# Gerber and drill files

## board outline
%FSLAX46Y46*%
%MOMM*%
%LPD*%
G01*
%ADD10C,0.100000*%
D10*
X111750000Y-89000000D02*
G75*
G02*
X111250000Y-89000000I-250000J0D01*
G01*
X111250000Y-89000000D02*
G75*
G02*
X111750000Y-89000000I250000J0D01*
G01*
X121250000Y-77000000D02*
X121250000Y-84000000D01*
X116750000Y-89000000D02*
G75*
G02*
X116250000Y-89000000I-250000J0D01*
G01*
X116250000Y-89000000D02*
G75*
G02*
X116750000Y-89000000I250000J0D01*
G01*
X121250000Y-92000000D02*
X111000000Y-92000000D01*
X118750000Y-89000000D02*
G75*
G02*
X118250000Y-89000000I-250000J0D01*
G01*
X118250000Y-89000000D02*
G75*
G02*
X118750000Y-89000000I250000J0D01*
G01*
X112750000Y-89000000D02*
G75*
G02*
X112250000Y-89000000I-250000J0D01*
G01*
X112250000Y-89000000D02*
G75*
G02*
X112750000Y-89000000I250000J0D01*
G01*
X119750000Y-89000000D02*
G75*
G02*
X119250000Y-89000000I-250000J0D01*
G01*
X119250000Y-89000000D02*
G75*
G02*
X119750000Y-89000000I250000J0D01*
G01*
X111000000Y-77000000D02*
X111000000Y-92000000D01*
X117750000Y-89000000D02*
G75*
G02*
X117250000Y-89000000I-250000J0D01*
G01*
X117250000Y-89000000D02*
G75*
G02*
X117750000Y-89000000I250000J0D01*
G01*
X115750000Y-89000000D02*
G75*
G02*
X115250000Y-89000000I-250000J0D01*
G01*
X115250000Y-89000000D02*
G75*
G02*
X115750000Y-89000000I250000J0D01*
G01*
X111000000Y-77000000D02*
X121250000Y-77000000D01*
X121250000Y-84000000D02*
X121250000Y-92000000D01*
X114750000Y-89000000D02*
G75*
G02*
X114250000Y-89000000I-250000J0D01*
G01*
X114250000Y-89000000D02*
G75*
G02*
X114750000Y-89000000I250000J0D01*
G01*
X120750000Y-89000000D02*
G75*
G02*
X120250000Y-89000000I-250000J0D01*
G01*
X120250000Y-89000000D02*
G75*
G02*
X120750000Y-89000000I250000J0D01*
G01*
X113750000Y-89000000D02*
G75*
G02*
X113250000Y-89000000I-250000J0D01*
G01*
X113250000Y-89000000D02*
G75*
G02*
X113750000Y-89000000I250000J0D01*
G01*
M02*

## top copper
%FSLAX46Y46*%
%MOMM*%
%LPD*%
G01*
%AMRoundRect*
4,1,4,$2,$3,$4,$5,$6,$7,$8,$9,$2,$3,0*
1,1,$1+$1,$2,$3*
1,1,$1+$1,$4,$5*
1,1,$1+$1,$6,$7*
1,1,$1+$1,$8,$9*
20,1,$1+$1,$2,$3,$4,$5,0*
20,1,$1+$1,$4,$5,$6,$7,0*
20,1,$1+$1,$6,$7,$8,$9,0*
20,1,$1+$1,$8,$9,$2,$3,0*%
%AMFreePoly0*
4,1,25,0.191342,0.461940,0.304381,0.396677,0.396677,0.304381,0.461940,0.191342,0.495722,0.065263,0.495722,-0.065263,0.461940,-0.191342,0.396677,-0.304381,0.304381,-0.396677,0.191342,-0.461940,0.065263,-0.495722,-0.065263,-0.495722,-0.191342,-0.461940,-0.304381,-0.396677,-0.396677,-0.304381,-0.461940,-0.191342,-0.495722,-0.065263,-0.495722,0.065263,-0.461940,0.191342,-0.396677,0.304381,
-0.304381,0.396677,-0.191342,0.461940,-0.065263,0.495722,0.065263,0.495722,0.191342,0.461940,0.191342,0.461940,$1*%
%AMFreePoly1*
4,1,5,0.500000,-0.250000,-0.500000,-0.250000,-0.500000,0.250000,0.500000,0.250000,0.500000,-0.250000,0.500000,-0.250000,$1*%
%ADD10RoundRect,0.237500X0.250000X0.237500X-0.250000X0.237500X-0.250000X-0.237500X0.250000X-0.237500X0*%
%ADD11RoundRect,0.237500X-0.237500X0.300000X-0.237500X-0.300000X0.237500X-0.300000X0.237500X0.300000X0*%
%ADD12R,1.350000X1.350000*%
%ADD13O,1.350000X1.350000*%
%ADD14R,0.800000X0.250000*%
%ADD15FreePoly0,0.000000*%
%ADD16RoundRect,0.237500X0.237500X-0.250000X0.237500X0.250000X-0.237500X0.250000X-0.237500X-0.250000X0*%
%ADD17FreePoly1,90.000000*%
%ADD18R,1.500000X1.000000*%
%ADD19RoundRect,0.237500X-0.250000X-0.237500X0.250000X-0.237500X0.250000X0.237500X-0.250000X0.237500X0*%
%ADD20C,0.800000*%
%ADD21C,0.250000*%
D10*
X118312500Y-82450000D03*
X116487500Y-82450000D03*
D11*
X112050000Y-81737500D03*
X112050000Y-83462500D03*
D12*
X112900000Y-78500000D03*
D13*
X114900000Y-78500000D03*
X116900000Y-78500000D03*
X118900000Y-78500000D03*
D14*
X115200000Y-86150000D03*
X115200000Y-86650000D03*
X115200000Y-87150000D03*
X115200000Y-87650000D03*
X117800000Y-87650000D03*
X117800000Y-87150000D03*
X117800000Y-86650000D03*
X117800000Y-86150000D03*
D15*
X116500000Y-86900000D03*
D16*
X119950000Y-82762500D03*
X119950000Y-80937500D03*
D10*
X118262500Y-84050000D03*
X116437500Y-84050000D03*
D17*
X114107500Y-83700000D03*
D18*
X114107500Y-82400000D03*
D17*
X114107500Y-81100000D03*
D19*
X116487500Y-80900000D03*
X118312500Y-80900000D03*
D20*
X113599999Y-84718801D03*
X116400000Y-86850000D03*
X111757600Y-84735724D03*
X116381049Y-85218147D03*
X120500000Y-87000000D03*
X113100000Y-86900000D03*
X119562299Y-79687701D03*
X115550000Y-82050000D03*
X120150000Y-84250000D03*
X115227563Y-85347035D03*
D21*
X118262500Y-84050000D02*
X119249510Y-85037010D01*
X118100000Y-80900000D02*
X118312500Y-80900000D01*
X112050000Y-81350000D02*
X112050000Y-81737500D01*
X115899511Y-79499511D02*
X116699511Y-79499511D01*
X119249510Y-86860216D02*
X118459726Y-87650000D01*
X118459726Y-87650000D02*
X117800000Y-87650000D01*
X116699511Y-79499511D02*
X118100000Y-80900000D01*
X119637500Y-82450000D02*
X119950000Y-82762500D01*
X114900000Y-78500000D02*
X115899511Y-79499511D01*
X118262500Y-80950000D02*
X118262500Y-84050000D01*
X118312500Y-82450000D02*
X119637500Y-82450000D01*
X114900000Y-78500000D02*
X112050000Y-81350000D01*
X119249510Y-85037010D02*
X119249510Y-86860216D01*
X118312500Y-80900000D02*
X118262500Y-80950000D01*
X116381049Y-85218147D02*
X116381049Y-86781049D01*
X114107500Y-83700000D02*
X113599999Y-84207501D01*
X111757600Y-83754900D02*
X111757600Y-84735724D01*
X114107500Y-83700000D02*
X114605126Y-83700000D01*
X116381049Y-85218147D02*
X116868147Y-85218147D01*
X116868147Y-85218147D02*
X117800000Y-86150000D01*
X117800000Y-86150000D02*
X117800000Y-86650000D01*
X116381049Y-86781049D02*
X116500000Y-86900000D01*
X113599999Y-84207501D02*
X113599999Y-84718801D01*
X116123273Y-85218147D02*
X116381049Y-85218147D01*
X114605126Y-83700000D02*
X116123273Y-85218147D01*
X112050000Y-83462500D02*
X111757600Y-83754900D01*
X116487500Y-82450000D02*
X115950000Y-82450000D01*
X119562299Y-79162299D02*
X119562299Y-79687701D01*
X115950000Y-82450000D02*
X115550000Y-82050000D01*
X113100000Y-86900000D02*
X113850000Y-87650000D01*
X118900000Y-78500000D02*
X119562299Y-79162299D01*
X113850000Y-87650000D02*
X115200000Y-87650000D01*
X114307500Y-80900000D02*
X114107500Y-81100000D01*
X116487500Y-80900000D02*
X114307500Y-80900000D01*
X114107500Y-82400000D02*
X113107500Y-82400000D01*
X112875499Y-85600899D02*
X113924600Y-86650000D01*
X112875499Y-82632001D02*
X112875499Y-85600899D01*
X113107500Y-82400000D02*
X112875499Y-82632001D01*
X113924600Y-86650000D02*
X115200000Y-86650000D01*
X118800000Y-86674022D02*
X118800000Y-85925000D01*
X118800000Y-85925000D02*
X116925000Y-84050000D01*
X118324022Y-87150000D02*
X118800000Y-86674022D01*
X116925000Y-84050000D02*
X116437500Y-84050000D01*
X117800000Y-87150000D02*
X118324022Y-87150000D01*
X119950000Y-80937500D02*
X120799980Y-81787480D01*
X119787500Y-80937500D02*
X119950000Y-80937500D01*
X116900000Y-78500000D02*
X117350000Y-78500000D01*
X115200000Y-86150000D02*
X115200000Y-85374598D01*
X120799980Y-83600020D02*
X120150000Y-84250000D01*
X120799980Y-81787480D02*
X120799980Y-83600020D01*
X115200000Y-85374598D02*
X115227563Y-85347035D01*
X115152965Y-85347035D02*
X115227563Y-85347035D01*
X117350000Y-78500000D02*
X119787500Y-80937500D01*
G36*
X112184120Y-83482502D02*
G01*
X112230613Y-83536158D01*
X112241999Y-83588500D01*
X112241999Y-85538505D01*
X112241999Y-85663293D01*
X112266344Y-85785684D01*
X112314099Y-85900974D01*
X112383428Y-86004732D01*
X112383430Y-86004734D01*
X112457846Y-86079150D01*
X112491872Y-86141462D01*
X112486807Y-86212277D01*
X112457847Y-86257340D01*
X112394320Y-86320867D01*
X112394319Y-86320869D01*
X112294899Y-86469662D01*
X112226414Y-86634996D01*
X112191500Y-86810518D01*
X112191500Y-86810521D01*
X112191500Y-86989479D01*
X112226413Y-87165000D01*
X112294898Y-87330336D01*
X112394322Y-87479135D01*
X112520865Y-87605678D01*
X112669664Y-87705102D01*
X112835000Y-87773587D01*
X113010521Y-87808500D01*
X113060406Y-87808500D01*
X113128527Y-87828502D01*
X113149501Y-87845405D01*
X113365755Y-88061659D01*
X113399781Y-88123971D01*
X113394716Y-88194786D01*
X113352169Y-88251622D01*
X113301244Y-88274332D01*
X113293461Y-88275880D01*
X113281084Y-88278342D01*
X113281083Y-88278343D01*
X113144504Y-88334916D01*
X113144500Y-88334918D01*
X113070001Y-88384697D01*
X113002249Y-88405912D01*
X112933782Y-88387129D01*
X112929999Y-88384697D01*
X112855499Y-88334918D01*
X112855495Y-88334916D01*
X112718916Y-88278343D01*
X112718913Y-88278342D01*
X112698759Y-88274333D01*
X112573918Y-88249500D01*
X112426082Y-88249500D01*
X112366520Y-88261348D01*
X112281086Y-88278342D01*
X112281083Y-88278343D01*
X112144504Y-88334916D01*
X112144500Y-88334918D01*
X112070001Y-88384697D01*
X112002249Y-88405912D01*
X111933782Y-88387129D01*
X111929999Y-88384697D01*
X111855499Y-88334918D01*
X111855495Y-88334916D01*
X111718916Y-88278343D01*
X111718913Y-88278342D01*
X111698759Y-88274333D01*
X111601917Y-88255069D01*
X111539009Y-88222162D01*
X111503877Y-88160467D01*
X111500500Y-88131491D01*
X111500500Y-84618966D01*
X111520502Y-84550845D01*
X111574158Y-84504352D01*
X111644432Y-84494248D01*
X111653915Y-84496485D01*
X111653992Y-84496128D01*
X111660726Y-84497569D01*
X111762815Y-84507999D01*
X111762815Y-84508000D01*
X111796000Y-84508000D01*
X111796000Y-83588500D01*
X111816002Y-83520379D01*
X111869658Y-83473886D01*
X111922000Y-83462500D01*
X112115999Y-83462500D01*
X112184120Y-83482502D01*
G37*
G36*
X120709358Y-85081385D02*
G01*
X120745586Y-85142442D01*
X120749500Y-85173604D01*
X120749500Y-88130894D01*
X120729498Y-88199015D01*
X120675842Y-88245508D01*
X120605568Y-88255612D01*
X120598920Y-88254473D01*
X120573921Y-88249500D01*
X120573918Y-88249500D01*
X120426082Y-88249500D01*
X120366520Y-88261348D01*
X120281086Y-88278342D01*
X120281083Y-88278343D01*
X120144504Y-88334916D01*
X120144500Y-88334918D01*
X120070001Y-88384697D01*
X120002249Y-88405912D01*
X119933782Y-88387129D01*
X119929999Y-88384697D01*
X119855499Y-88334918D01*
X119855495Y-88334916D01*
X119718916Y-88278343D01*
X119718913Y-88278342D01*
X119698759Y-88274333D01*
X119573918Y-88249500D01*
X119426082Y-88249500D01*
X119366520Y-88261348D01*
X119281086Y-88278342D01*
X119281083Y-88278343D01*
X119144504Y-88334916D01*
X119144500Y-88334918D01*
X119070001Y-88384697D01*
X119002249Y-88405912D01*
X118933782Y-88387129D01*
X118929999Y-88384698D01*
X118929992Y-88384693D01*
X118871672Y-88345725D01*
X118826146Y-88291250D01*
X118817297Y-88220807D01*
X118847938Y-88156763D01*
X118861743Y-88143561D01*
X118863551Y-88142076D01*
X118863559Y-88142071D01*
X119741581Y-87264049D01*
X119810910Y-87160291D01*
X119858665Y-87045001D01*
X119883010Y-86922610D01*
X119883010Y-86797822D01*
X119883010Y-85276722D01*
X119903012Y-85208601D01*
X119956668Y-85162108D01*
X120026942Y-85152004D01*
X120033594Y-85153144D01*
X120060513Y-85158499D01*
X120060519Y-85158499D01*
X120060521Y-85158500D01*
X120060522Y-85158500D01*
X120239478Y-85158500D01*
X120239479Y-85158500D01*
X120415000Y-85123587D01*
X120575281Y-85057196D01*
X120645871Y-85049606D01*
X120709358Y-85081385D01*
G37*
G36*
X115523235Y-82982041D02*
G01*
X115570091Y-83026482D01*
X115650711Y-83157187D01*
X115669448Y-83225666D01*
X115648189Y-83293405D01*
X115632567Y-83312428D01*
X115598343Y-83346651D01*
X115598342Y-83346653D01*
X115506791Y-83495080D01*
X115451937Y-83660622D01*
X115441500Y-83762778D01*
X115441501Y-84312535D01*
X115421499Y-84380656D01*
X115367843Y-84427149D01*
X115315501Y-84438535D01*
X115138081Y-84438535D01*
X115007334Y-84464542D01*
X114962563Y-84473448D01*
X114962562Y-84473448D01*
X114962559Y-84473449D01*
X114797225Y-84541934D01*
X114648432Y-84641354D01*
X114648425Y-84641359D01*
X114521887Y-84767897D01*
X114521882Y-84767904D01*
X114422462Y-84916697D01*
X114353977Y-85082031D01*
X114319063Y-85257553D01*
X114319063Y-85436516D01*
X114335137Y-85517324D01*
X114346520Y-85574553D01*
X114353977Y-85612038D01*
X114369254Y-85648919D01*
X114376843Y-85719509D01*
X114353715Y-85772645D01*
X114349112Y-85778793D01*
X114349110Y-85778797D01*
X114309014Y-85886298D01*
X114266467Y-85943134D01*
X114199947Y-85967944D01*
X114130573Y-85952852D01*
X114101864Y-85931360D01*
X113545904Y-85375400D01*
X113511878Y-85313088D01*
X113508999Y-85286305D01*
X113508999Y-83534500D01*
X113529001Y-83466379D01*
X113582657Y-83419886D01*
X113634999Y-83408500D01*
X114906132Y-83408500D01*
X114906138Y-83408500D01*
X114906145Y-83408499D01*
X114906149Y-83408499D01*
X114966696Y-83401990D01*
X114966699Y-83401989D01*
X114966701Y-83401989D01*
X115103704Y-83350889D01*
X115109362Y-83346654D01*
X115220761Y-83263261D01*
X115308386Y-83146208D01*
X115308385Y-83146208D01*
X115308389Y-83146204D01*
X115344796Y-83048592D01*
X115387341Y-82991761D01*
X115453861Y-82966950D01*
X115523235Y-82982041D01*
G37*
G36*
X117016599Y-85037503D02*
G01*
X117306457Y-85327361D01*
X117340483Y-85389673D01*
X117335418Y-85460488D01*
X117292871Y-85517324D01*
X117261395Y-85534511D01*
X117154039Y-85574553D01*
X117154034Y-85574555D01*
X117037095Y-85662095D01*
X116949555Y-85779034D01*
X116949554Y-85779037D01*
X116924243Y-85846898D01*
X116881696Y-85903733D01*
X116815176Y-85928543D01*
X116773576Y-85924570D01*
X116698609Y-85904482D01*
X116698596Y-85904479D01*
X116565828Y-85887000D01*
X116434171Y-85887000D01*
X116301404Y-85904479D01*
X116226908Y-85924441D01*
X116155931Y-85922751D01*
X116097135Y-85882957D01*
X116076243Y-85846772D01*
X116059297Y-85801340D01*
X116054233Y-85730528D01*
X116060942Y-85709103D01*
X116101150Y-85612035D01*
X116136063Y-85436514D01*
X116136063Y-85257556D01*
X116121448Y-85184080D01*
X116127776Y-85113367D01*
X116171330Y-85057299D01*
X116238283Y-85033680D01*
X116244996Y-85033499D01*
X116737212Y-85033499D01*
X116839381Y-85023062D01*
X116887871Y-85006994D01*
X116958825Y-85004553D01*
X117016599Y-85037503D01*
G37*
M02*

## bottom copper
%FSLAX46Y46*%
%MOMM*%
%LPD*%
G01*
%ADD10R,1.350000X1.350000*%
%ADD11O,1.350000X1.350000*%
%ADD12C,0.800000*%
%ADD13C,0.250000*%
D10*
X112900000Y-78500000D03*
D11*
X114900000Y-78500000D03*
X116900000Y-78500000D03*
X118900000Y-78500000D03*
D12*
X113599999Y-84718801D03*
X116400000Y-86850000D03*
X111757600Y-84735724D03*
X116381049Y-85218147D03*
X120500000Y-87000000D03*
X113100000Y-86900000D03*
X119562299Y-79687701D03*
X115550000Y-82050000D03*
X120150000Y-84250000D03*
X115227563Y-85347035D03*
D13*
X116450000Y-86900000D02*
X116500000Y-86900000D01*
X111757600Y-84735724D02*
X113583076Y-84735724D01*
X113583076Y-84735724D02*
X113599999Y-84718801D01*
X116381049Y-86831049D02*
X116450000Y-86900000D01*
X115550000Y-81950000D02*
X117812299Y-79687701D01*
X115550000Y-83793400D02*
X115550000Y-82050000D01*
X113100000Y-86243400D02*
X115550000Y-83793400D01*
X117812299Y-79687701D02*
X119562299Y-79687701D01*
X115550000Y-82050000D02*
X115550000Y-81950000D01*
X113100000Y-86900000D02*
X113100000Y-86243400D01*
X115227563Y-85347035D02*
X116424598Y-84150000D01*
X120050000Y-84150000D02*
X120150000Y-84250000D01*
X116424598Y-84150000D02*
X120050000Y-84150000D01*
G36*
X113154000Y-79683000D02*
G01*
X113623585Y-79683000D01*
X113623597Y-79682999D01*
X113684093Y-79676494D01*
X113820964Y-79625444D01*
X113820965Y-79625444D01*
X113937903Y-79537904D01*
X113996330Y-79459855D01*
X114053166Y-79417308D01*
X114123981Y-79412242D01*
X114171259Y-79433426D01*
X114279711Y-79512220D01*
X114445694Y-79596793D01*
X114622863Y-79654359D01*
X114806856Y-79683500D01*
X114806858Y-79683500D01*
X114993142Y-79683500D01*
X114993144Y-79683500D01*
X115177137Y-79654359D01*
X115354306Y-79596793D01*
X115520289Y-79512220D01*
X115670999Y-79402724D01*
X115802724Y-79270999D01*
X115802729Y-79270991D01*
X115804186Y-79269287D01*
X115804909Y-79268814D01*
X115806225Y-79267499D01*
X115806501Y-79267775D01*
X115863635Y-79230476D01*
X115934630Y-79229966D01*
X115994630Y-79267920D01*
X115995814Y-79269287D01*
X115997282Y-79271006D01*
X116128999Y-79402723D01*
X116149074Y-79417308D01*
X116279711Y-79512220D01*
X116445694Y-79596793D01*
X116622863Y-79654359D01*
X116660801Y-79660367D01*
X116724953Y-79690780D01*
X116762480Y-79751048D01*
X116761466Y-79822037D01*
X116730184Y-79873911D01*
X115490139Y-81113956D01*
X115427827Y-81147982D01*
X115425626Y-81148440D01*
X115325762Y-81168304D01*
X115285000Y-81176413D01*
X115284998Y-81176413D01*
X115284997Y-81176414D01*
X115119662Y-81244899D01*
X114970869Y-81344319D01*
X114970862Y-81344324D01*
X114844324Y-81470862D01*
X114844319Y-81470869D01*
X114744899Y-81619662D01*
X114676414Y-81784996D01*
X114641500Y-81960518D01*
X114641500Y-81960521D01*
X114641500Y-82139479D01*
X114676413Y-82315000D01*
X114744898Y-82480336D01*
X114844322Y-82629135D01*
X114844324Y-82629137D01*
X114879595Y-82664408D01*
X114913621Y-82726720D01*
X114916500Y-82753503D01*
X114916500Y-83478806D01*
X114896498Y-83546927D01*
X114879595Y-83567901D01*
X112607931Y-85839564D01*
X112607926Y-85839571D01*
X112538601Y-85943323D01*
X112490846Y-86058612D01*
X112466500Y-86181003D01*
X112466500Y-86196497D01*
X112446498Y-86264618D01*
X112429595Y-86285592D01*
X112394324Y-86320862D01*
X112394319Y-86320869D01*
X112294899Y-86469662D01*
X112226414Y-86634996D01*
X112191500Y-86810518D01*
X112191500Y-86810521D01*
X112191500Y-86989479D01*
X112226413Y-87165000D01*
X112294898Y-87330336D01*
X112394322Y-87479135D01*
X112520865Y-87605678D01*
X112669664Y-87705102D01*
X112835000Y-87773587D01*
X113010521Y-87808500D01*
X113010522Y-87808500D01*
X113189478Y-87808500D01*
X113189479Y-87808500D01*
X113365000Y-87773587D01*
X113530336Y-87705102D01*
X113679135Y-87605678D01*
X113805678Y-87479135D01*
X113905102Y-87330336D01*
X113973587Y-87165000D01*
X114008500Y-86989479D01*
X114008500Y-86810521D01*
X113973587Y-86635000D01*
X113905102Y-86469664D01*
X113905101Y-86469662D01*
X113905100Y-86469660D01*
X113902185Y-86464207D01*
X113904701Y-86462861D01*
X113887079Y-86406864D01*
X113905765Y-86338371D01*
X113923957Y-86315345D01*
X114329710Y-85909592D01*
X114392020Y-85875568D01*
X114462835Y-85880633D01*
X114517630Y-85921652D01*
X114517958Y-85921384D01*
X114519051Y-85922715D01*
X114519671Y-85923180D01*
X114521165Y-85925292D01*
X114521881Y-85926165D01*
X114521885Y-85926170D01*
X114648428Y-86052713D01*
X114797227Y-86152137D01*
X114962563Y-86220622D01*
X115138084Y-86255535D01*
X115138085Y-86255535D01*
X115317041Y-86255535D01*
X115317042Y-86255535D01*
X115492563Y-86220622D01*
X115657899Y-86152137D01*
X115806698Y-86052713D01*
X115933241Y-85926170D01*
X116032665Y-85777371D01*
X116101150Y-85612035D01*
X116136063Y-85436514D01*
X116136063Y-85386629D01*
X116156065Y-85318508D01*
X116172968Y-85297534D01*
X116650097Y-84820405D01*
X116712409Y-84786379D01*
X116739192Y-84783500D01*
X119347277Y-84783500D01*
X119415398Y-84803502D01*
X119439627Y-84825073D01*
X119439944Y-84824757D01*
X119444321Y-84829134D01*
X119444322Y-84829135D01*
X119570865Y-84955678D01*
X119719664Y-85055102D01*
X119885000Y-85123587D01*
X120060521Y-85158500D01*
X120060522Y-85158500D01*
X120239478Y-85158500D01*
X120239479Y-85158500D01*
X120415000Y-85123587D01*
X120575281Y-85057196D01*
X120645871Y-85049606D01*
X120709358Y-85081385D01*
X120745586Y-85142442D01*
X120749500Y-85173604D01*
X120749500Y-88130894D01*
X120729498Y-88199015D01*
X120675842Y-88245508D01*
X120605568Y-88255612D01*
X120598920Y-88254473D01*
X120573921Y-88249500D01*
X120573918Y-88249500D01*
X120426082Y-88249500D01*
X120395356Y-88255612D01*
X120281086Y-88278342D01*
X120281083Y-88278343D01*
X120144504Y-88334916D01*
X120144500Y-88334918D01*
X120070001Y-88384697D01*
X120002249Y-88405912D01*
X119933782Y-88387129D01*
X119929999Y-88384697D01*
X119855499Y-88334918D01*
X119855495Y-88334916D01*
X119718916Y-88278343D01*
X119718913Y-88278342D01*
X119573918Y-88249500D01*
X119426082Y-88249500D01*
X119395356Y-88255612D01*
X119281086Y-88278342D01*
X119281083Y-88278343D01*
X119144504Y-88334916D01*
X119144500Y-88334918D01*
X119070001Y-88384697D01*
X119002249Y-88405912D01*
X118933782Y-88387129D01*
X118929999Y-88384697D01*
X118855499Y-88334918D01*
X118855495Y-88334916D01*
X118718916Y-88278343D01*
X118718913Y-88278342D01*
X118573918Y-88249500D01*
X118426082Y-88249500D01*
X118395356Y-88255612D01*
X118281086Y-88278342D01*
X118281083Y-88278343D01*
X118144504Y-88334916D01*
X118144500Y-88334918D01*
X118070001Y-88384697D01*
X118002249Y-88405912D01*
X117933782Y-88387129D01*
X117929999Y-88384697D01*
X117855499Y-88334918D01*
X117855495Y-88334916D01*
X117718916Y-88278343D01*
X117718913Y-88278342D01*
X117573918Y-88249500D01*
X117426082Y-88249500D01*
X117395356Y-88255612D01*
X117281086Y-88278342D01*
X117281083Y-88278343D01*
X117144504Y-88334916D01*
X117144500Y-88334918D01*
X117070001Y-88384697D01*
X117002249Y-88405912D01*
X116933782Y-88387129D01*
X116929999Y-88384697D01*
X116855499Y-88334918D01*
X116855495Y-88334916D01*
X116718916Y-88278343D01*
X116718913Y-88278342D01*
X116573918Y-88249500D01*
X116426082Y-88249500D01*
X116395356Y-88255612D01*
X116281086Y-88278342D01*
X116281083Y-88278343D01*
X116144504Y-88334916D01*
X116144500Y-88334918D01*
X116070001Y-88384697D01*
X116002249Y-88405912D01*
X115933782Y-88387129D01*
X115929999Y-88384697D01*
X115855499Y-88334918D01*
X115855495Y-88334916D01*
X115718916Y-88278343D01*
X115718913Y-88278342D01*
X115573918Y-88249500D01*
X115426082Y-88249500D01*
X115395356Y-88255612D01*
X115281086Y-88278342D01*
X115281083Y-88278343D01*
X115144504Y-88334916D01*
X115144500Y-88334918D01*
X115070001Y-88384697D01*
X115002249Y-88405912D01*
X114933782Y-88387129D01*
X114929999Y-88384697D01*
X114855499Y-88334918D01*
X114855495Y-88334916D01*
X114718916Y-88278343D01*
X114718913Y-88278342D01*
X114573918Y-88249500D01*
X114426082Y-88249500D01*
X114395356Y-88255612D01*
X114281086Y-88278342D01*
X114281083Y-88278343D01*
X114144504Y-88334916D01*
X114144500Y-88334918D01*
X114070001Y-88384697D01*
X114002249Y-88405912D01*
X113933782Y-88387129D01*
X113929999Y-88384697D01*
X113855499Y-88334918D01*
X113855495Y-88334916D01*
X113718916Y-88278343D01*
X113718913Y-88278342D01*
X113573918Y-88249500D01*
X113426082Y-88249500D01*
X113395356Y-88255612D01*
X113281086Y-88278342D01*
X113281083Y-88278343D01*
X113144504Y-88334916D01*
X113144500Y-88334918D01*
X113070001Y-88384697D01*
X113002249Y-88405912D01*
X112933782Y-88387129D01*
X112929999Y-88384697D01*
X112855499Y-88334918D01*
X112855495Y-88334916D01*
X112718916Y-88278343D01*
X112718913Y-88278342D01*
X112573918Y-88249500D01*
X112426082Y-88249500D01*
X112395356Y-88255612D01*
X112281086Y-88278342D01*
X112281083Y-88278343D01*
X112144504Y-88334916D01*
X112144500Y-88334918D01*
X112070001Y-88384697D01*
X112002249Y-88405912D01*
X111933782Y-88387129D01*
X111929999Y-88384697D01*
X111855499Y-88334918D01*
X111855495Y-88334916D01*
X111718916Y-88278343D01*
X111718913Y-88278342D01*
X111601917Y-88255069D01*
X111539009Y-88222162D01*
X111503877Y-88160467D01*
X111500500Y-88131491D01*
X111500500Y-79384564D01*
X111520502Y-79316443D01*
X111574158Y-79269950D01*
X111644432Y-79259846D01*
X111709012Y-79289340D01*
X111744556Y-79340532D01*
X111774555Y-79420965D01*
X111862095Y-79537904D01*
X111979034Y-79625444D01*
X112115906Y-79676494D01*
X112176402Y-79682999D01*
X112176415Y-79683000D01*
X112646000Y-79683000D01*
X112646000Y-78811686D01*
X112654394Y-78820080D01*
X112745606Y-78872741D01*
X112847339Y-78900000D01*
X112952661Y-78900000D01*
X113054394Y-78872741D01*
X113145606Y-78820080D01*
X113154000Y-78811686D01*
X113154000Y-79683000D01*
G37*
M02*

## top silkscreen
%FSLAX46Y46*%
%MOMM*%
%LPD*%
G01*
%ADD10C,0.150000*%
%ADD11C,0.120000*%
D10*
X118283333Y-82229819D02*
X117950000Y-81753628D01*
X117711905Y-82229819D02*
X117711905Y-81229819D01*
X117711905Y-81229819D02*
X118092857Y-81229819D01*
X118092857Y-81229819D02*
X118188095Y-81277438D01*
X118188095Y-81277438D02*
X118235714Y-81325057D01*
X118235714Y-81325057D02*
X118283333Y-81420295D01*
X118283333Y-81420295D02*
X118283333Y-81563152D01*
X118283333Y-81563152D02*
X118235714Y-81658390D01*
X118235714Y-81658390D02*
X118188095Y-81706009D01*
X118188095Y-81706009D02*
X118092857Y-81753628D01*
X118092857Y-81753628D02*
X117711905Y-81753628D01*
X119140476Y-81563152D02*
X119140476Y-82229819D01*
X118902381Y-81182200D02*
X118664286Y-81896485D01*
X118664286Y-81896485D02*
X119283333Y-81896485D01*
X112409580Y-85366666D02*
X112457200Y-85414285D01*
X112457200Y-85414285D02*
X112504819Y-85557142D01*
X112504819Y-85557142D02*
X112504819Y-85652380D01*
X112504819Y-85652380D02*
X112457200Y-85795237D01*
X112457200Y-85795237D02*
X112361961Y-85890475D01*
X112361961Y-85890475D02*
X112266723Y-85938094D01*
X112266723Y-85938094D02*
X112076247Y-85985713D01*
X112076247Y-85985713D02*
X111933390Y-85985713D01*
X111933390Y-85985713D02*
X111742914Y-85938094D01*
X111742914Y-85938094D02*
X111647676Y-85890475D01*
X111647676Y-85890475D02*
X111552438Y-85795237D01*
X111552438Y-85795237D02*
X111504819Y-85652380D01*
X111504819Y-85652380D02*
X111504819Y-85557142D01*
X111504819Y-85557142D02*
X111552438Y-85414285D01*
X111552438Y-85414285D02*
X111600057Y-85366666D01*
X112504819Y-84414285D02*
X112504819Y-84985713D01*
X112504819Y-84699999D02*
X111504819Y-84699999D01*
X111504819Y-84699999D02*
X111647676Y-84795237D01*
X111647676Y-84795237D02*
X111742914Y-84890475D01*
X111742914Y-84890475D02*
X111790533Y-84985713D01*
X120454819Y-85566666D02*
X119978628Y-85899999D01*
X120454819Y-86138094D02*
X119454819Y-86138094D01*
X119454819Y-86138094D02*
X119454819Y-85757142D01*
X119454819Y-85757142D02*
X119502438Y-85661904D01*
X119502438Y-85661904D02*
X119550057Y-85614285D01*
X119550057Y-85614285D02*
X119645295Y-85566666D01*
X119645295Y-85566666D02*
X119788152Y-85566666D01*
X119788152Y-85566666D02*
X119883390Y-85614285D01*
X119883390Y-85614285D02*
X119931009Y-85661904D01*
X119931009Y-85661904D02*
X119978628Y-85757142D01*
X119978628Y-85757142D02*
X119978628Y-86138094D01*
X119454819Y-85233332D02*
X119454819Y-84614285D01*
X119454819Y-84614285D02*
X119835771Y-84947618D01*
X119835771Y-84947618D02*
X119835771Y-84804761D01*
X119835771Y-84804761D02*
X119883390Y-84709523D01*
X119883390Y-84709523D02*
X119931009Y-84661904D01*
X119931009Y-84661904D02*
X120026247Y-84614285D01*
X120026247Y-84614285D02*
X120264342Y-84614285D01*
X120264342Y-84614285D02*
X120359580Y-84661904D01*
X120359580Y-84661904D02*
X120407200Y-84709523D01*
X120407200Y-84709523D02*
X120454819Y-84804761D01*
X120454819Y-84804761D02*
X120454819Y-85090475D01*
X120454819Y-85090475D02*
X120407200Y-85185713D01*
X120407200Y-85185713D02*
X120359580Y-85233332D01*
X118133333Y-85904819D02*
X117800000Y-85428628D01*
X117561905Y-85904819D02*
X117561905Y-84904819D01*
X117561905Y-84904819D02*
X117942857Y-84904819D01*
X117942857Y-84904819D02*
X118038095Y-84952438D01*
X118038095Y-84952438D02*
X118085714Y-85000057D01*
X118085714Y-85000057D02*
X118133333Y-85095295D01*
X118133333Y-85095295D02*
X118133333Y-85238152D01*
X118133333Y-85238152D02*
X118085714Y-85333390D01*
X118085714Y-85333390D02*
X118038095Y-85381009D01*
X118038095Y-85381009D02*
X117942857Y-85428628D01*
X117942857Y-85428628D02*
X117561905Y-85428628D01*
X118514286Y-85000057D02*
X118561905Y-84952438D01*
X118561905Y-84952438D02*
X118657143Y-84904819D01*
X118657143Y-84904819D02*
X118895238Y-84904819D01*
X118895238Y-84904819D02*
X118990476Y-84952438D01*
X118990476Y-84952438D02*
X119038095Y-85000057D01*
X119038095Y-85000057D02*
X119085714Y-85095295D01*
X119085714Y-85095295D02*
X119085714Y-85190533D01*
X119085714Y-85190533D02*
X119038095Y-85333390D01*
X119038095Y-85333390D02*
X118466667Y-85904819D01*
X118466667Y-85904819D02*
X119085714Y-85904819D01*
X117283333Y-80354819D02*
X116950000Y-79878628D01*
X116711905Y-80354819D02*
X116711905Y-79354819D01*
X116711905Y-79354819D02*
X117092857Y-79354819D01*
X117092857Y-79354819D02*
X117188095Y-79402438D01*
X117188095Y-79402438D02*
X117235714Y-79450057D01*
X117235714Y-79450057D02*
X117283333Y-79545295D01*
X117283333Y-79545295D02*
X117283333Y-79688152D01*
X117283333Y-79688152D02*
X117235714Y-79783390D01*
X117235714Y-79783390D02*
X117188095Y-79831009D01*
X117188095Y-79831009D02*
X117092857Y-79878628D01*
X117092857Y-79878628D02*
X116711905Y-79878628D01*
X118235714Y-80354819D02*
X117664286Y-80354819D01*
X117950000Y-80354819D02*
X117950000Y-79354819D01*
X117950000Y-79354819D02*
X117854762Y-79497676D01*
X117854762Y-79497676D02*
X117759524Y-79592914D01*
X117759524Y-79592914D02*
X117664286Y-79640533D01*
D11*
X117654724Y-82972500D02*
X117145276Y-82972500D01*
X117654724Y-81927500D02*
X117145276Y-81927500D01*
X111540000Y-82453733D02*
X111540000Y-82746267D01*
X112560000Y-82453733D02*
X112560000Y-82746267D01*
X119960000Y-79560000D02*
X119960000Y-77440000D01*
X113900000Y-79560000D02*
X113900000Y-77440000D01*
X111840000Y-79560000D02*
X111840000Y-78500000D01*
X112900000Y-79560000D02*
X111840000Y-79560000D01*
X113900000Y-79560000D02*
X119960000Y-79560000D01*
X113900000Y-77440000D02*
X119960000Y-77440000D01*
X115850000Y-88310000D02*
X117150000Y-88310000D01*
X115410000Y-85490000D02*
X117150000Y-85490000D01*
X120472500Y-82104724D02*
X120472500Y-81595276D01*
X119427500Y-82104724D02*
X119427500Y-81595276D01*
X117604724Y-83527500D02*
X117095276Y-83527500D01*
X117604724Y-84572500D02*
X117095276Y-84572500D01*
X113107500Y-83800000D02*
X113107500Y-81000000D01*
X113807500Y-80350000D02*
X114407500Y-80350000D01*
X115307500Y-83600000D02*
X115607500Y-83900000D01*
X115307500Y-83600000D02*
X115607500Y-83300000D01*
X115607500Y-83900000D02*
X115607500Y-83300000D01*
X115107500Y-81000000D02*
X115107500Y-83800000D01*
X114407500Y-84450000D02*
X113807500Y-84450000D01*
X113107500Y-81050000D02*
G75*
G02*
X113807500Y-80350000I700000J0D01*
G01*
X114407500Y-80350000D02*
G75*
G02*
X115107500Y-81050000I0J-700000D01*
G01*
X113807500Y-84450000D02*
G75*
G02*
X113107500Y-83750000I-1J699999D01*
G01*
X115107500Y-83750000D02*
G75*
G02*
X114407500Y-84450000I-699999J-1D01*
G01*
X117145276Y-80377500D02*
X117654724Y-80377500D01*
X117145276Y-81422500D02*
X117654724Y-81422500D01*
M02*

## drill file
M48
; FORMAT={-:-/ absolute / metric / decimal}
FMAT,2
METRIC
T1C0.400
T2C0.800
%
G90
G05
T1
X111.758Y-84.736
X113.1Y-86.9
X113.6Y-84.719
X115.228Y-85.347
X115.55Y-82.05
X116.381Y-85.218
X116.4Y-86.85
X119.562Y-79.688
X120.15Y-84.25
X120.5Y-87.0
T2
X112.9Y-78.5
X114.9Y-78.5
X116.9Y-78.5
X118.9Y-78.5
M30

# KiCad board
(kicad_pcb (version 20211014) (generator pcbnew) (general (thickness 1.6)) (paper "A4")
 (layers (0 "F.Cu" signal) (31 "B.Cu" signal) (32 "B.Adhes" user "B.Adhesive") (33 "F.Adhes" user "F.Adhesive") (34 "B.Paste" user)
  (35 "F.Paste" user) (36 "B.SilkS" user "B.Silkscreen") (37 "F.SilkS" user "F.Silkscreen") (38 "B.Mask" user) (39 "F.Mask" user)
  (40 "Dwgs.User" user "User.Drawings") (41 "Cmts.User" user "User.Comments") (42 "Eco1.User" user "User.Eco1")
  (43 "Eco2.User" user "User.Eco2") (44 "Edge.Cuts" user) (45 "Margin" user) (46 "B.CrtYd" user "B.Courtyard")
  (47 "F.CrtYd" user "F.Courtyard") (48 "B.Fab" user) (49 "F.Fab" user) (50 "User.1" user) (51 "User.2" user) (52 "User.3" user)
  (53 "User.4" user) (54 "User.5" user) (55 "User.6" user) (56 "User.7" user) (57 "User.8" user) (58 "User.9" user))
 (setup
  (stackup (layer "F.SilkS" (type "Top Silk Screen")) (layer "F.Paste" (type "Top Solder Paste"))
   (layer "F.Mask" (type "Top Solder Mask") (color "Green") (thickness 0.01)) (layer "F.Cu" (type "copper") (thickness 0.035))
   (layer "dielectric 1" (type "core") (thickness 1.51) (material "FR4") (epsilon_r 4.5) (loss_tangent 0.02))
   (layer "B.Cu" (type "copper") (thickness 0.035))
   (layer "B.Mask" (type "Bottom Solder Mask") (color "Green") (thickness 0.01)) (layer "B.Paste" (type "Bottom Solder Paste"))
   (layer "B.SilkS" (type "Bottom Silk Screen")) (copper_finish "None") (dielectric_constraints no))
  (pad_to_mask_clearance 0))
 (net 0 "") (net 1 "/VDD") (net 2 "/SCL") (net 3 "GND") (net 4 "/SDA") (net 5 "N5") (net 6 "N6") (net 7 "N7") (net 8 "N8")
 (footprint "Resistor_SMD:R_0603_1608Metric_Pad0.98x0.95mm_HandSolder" (layer "F.Cu") (at 117.4 82.45 180)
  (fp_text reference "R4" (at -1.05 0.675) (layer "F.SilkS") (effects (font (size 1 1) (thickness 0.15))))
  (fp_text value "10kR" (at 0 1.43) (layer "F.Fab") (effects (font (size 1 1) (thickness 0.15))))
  (fp_line (start -0.254724 -0.5225) (end 0.254724 -0.5225) (layer "F.SilkS") (width 0.12))
  (fp_line (start -0.254724 0.5225) (end 0.254724 0.5225) (layer "F.SilkS") (width 0.12))
  (pad "1" smd roundrect locked (at -0.9125 0 180) (size 0.975 0.95) (layers "F.Cu" "F.Paste" "F.Mask") (roundrect_rratio 0.25)
   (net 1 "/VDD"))
  (pad "2" smd roundrect locked (at 0.9125 0 180) (size 0.975 0.95) (layers "F.Cu" "F.Paste" "F.Mask") (roundrect_rratio 0.25)
   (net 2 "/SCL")))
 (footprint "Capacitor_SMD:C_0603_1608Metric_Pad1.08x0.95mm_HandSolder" (layer "F.Cu") (at 112.05 82.6 -90)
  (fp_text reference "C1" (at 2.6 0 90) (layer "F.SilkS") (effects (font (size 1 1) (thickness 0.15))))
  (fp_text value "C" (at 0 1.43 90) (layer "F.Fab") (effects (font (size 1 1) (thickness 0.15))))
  (fp_line (start -0.146267 0.51) (end 0.146267 0.51) (layer "F.SilkS") (width 0.12))
  (fp_line (start -0.146267 -0.51) (end 0.146267 -0.51) (layer "F.SilkS") (width 0.12))
  (pad "1" smd roundrect locked (at -0.8625 0 270) (size 1.075 0.95) (layers "F.Cu" "F.Paste" "F.Mask") (roundrect_rratio 0.25)
   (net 1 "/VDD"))
  (pad "2" smd roundrect locked (at 0.8625 0 270) (size 1.075 0.95) (layers "F.Cu" "F.Paste" "F.Mask") (roundrect_rratio 0.25) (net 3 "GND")))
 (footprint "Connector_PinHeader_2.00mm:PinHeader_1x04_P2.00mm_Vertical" (layer "F.Cu") (at 112.9 78.5 90)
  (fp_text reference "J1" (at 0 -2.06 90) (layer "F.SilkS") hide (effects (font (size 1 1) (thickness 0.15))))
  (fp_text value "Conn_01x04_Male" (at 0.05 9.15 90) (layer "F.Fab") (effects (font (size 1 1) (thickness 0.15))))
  (fp_line (start -1.06 7.06) (end 1.06 7.06) (layer "F.SilkS") (width 0.12))
  (fp_line (start -1.06 1) (end 1.06 1) (layer "F.SilkS") (width 0.12))
  (fp_line (start -1.06 -1.06) (end 0 -1.06) (layer "F.SilkS") (width 0.12))
  (fp_line (start -1.06 0) (end -1.06 -1.06) (layer "F.SilkS") (width 0.12))
  (fp_line (start -1.06 1) (end -1.06 7.06) (layer "F.SilkS") (width 0.12))
  (fp_line (start 1.06 1) (end 1.06 7.06) (layer "F.SilkS") (width 0.12))
  (pad "1" thru_hole rect locked (at 0 0 90) (size 1.35 1.35) (drill 0.8) (layers *.Cu *.Mask) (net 3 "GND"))
  (pad "2" thru_hole oval locked (at 0 2 90) (size 1.35 1.35) (drill 0.8) (layers *.Cu *.Mask) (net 1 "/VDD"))
  (pad "3" thru_hole oval locked (at 0 4 90) (size 1.35 1.35) (drill 0.8) (layers *.Cu *.Mask) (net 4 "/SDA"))
  (pad "4" thru_hole oval locked (at 0 6 90) (size 1.35 1.35) (drill 0.8) (layers *.Cu *.Mask) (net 2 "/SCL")))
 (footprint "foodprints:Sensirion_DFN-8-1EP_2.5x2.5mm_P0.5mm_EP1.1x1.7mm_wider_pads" (layer "F.Cu") (at 116.5 86.9)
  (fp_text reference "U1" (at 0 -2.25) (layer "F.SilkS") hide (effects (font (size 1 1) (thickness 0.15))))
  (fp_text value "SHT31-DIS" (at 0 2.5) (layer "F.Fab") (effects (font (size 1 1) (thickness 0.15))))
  (fp_line (start -0.65 1.41) (end 0.65 1.41) (layer "F.SilkS") (width 0.12))
  (fp_line (start -1.09 -1.41) (end 0.65 -1.41) (layer "F.SilkS") (width 0.12))
  (pad "" smd custom locked (at 0 0) (size 0.9 0.9) (layers "F.Paste") (zone_connect 0) (options (clearance outline) (anchor rect))
   (primitives))
  (pad "1" smd rect locked (at -1.3 -0.75) (size 0.8 0.25) (layers "F.Cu" "F.Paste" "F.Mask") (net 4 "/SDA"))
  (pad "2" smd rect locked (at -1.3 -0.25) (size 0.8 0.25) (layers "F.Cu" "F.Paste" "F.Mask") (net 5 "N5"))
  (pad "3" smd rect locked (at -1.3 0.25) (size 0.8 0.25) (layers "F.Cu" "F.Paste" "F.Mask") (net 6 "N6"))
  (pad "4" smd rect locked (at -1.3 0.75) (size 0.8 0.25) (layers "F.Cu" "F.Paste" "F.Mask") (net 2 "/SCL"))
  (pad "5" smd rect locked (at 1.3 0.75) (size 0.8 0.25) (layers "F.Cu" "F.Paste" "F.Mask") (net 1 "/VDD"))
  (pad "6" smd rect locked (at 1.3 0.25) (size 0.8 0.25) (layers "F.Cu" "F.Paste" "F.Mask") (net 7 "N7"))
  (pad "7" smd rect locked (at 1.3 -0.25) (size 0.8 0.25) (layers "F.Cu" "F.Paste" "F.Mask") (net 3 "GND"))
  (pad "8" smd rect locked (at 1.3 -0.75) (size 0.8 0.25) (layers "F.Cu" "F.Paste" "F.Mask") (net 3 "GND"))
  (pad "9" smd custom locked (at 0 0) (size 1 1) (layers "F.Cu" "F.Mask") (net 3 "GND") (zone_connect 0)
   (options (clearance outline) (anchor circle)) (primitives)))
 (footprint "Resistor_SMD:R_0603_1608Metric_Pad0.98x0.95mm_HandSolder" (layer "F.Cu") (at 119.95 81.85 90)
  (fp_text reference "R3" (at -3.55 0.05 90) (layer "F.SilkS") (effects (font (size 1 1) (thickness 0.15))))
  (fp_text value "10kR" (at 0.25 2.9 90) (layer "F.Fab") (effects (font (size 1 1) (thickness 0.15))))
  (fp_line (start -0.254724 0.5225) (end 0.254724 0.5225) (layer "F.SilkS") (width 0.12))
  (fp_line (start -0.254724 -0.5225) (end 0.254724 -0.5225) (layer "F.SilkS") (width 0.12))
  (pad "1" smd roundrect locked (at -0.9125 0 90) (size 0.975 0.95) (layers "F.Cu" "F.Paste" "F.Mask") (roundrect_rratio 0.25)
   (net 1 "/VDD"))
  (pad "2" smd roundrect locked (at 0.9125 0 90) (size 0.975 0.95) (layers "F.Cu" "F.Paste" "F.Mask") (roundrect_rratio 0.25) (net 4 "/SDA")))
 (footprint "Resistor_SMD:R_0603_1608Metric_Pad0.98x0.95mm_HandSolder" (layer "F.Cu") (at 117.35 84.05 180)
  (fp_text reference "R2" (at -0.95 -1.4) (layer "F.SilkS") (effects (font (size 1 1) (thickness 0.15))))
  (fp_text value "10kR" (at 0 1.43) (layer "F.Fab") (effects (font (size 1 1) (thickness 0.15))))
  (fp_line (start -0.254724 0.5225) (end 0.254724 0.5225) (layer "F.SilkS") (width 0.12))
  (fp_line (start -0.254724 -0.5225) (end 0.254724 -0.5225) (layer "F.SilkS") (width 0.12))
  (pad "1" smd roundrect locked (at -0.9125 0 180) (size 0.975 0.95) (layers "F.Cu" "F.Paste" "F.Mask") (roundrect_rratio 0.25)
   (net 1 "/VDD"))
  (pad "2" smd roundrect locked (at 0.9125 0 180) (size 0.975 0.95) (layers "F.Cu" "F.Paste" "F.Mask") (roundrect_rratio 0.25) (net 7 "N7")))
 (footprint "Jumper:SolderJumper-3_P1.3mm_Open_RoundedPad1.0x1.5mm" (layer "F.Cu") (at 114.1075 82.4 90)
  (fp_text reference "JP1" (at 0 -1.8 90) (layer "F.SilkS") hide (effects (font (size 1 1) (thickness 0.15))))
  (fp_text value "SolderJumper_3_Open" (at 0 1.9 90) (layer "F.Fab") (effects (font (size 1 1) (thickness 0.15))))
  (fp_line (start -1.4 -1) (end 1.4 -1) (layer "F.SilkS") (width 0.12))
  (fp_line (start 2.05 -0.3) (end 2.05 0.3) (layer "F.SilkS") (width 0.12))
  (fp_line (start -1.2 1.2) (end -1.5 1.5) (layer "F.SilkS") (width 0.12))
  (fp_line (start -1.2 1.2) (end -0.9 1.5) (layer "F.SilkS") (width 0.12))
  (fp_line (start -1.5 1.5) (end -0.9 1.5) (layer "F.SilkS") (width 0.12))
  (fp_line (start 1.4 1) (end -1.4 1) (layer "F.SilkS") (width 0.12))
  (fp_line (start -2.05 0.3) (end -2.05 -0.3) (layer "F.SilkS") (width 0.12))
  (fp_arc (start 1.35 -1) (mid 1.844975 -0.794975) (end 2.05 -0.3) (layer "F.SilkS") (width 0.12))
  (fp_arc (start 2.05 0.3) (mid 1.844975 0.794975) (end 1.35 1) (layer "F.SilkS") (width 0.12))
  (fp_arc (start -2.05 -0.3) (mid -1.844975 -0.794975) (end -1.35 -1) (layer "F.SilkS") (width 0.12))
  (fp_arc (start -1.35 1) (mid -1.844975 0.794975) (end -2.05 0.3) (layer "F.SilkS") (width 0.12))
  (pad "1" smd custom locked (at -1.3 0 90) (size 1 0.5) (layers "F.Cu" "F.Mask") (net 3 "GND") (zone_connect 2)
   (options (clearance outline) (anchor rect)) (primitives))
  (pad "2" smd rect locked (at 0 0 90) (size 1 1.5) (layers "F.Cu" "F.Mask") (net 5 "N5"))
  (pad "3" smd custom locked (at 1.3 0 90) (size 1 0.5) (layers "F.Cu" "F.Mask") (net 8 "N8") (zone_connect 2)
   (options (clearance outline) (anchor rect)) (primitives)))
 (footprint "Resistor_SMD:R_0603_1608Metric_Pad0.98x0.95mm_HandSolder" (layer "F.Cu") (at 117.4 80.9)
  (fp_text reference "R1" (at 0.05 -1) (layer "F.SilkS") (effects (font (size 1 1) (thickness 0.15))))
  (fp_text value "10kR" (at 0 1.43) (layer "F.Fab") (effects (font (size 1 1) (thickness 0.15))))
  (fp_line (start -0.254724 -0.5225) (end 0.254724 -0.5225) (layer "F.SilkS") (width 0.12))
  (fp_line (start -0.254724 0.5225) (end 0.254724 0.5225) (layer "F.SilkS") (width 0.12))
  (pad "1" smd roundrect locked (at -0.9125 0) (size 0.975 0.95) (layers "F.Cu" "F.Paste" "F.Mask") (roundrect_rratio 0.25) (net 8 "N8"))
  (pad "2" smd roundrect locked (at 0.9125 0) (size 0.975 0.95) (layers "F.Cu" "F.Paste" "F.Mask") (roundrect_rratio 0.25) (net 1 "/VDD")))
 (gr_circle (center 111.5 89) (end 111.75 89) (layer "Edge.Cuts") (width 0.1) (fill none))
 (gr_line (start 121.25 77) (end 121.25 84) (layer "Edge.Cuts") (width 0.1))
 (gr_circle (center 116.5 89) (end 116.75 89) (layer "Edge.Cuts") (width 0.1) (fill none))
 (gr_line (start 121.25 92) (end 111 92) (layer "Edge.Cuts") (width 0.1))
 (gr_circle (center 118.5 89) (end 118.75 89) (layer "Edge.Cuts") (width 0.1) (fill none))
 (gr_circle (center 112.5 89) (end 112.75 89) (layer "Edge.Cuts") (width 0.1) (fill none))
 (gr_circle (center 119.5 89) (end 119.75 89) (layer "Edge.Cuts") (width 0.1) (fill none))
 (gr_line (start 111 77) (end 111 92) (layer "Edge.Cuts") (width 0.1))
 (gr_circle (center 117.5 89) (end 117.75 89) (layer "Edge.Cuts") (width 0.1) (fill none))
 (gr_circle (center 115.5 89) (end 115.75 89) (layer "Edge.Cuts") (width 0.1) (fill none))
 (gr_line (start 111 77) (end 121.25 77) (layer "Edge.Cuts") (width 0.1))
 (gr_line (start 121.25 84) (end 121.25 92) (layer "Edge.Cuts") (width 0.1))
 (gr_circle (center 114.5 89) (end 114.75 89) (layer "Edge.Cuts") (width 0.1) (fill none))
 (gr_circle (center 120.5 89) (end 120.75 89) (layer "Edge.Cuts") (width 0.1) (fill none))
 (gr_circle (center 113.5 89) (end 113.75 89) (layer "Edge.Cuts") (width 0.1) (fill none))
 (segment (start 118.2625 84.05) (end 119.24951 85.03701) (width 0.25) (layer "F.Cu") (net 1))
 (segment (start 118.1 80.9) (end 118.3125 80.9) (width 0.25) (layer "F.Cu") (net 1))
 (segment (start 112.05 81.35) (end 112.05 81.7375) (width 0.25) (layer "F.Cu") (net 1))
 (segment (start 115.899511 79.499511) (end 116.699511 79.499511) (width 0.25) (layer "F.Cu") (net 1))
 (segment (start 119.24951 86.860216) (end 118.459726 87.65) (width 0.25) (layer "F.Cu") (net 1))
 (segment (start 118.459726 87.65) (end 117.8 87.65) (width 0.25) (layer "F.Cu") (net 1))
 (segment (start 116.699511 79.499511) (end 118.1 80.9) (width 0.25) (layer "F.Cu") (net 1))
 (segment (start 119.6375 82.45) (end 119.95 82.7625) (width 0.25) (layer "F.Cu") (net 1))
 (segment (start 114.9 78.5) (end 115.899511 79.499511) (width 0.25) (layer "F.Cu") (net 1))
 (segment (start 118.2625 80.95) (end 118.2625 84.05) (width 0.25) (layer "F.Cu") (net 1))
 (segment (start 118.3125 82.45) (end 119.6375 82.45) (width 0.25) (layer "F.Cu") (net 1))
 (segment (start 114.9 78.5) (end 112.05 81.35) (width 0.25) (layer "F.Cu") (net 1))
 (segment (start 119.24951 85.03701) (end 119.24951 86.860216) (width 0.25) (layer "F.Cu") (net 1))
 (segment (start 118.3125 80.9) (end 118.2625 80.95) (width 0.25) (layer "F.Cu") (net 1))
 (segment (start 116.381049 85.218147) (end 116.381049 86.781049) (width 0.25) (layer "F.Cu") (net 3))
 (segment (start 114.1075 83.7) (end 113.599999 84.207501) (width 0.25) (layer "F.Cu") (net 3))
 (segment (start 111.7576 83.7549) (end 111.7576 84.735724) (width 0.25) (layer "F.Cu") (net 3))
 (segment (start 114.1075 83.7) (end 114.605126 83.7) (width 0.25) (layer "F.Cu") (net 3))
 (segment (start 116.381049 85.218147) (end 116.868147 85.218147) (width 0.25) (layer "F.Cu") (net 3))
 (segment (start 116.868147 85.218147) (end 117.8 86.15) (width 0.25) (layer "F.Cu") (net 3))
 (segment (start 117.8 86.15) (end 117.8 86.65) (width 0.25) (layer "F.Cu") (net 3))
 (segment (start 116.381049 86.781049) (end 116.5 86.9) (width 0.25) (layer "F.Cu") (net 3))
 (segment (start 113.599999 84.207501) (end 113.599999 84.718801) (width 0.25) (layer "F.Cu") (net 3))
 (segment (start 116.123273 85.218147) (end 116.381049 85.218147) (width 0.25) (layer "F.Cu") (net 3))
 (segment (start 114.605126 83.7) (end 116.123273 85.218147) (width 0.25) (layer "F.Cu") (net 3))
 (segment (start 112.05 83.4625) (end 111.7576 83.7549) (width 0.25) (layer "F.Cu") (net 3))
 (via (at 113.599999 84.718801) (size 0.8) (drill 0.4) (layers "F.Cu" "B.Cu") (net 3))
 (via (at 116.4 86.85) (size 0.8) (drill 0.4) (layers "F.Cu" "B.Cu") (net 3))
 (via (at 111.7576 84.735724) (size 0.8) (drill 0.4) (layers "F.Cu" "B.Cu") (free) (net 3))
 (via (at 116.381049 85.218147) (size 0.8) (drill 0.4) (layers "F.Cu" "B.Cu") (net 3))
 (via (at 120.5 87) (size 0.8) (drill 0.4) (layers "F.Cu" "B.Cu") (free) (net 3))
 (segment (start 116.45 86.9) (end 116.5 86.9) (width 0.25) (layer "B.Cu") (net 3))
 (segment (start 111.7576 84.735724) (end 113.583076 84.735724) (width 0.25) (layer "B.Cu") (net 3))
 (segment (start 113.583076 84.735724) (end 113.599999 84.718801) (width 0.25) (layer "B.Cu") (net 3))
 (segment (start 116.381049 86.831049) (end 116.45 86.9) (width 0.25) (layer "B.Cu") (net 3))
 (segment (start 116.4875 82.45) (end 115.95 82.45) (width 0.25) (layer "F.Cu") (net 2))
 (segment (start 119.562299 79.162299) (end 119.562299 79.687701) (width 0.25) (layer "F.Cu") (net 2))
 (segment (start 115.95 82.45) (end 115.55 82.05) (width 0.25) (layer "F.Cu") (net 2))
 (segment (start 113.1 86.9) (end 113.85 87.65) (width 0.25) (layer "F.Cu") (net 2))
 (segment (start 118.9 78.5) (end 119.562299 79.162299) (width 0.25) (layer "F.Cu") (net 2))
 (segment (start 113.85 87.65) (end 115.2 87.65) (width 0.25) (layer "F.Cu") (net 2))
 (via (at 113.1 86.9) (size 0.8) (drill 0.4) (layers "F.Cu" "B.Cu") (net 2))
 (via (at 119.562299 79.687701) (size 0.8) (drill 0.4) (layers "F.Cu" "B.Cu") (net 2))
 (via (at 115.55 82.05) (size 0.8) (drill 0.4) (layers "F.Cu" "B.Cu") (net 2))
 (segment (start 115.55 81.95) (end 117.812299 79.687701) (width 0.25) (layer "B.Cu") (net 2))
 (segment (start 115.55 83.7934) (end 115.55 82.05) (width 0.25) (layer "B.Cu") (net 2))
 (segment (start 113.1 86.2434) (end 115.55 83.7934) (width 0.25) (layer "B.Cu") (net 2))
 (segment (start 117.812299 79.687701) (end 119.562299 79.687701) (width 0.25) (layer "B.Cu") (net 2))
 (segment (start 115.55 82.05) (end 115.55 81.95) (width 0.25) (layer "B.Cu") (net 2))
 (segment (start 113.1 86.9) (end 113.1 86.2434) (width 0.25) (layer "B.Cu") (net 2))
 (segment (start 114.3075 80.9) (end 114.1075 81.1) (width 0.25) (layer "F.Cu") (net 8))
 (segment (start 116.4875 80.9) (end 114.3075 80.9) (width 0.25) (layer "F.Cu") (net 8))
 (segment (start 114.1075 82.4) (end 113.1075 82.4) (width 0.25) (layer "F.Cu") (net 5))
 (segment (start 112.875499 85.600899) (end 113.9246 86.65) (width 0.25) (layer "F.Cu") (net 5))
 (segment (start 112.875499 82.632001) (end 112.875499 85.600899) (width 0.25) (layer "F.Cu") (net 5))
 (segment (start 113.1075 82.4) (end 112.875499 82.632001) (width 0.25) (layer "F.Cu") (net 5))
 (segment (start 113.9246 86.65) (end 115.2 86.65) (width 0.25) (layer "F.Cu") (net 5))
 (segment (start 118.8 86.674022) (end 118.8 85.925) (width 0.25) (layer "F.Cu") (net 7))
 (segment (start 118.8 85.925) (end 116.925 84.05) (width 0.25) (layer "F.Cu") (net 7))
 (segment (start 118.324022 87.15) (end 118.8 86.674022) (width 0.25) (layer "F.Cu") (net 7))
 (segment (start 116.925 84.05) (end 116.4375 84.05) (width 0.25) (layer "F.Cu") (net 7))
 (segment (start 117.8 87.15) (end 118.324022 87.15) (width 0.25) (layer "F.Cu") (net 7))
 (segment (start 119.95 80.9375) (end 120.79998 81.78748) (width 0.25) (layer "F.Cu") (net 4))
 (segment (start 119.7875 80.9375) (end 119.95 80.9375) (width 0.25) (layer "F.Cu") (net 4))
 (segment (start 116.9 78.5) (end 117.35 78.5) (width 0.25) (layer "F.Cu") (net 4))
 (segment (start 115.2 86.15) (end 115.2 85.374598) (width 0.25) (layer "F.Cu") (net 4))
 (segment (start 120.79998 83.60002) (end 120.15 84.25) (width 0.25) (layer "F.Cu") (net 4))
 (segment (start 120.79998 81.78748) (end 120.79998 83.60002) (width 0.25) (layer "F.Cu") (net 4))
 (segment (start 115.2 85.374598) (end 115.227563 85.347035) (width 0.25) (layer "F.Cu") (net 4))
 (segment (start 115.152965 85.347035) (end 115.227563 85.347035) (width 0.25) (layer "F.Cu") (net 4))
 (segment (start 117.35 78.5) (end 119.7875 80.9375) (width 0.25) (layer "F.Cu") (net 4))
 (via (at 120.15 84.25) (size 0.8) (drill 0.4) (layers "F.Cu" "B.Cu") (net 4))
 (via (at 115.227563 85.347035) (size 0.8) (drill 0.4) (layers "F.Cu" "B.Cu") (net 4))
 (segment (start 115.227563 85.347035) (end 116.424598 84.15) (width 0.25) (layer "B.Cu") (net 4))
 (segment (start 120.05 84.15) (end 120.15 84.25) (width 0.25) (layer "B.Cu") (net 4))
 (segment (start 116.424598 84.15) (end 120.05 84.15) (width 0.25) (layer "B.Cu") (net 4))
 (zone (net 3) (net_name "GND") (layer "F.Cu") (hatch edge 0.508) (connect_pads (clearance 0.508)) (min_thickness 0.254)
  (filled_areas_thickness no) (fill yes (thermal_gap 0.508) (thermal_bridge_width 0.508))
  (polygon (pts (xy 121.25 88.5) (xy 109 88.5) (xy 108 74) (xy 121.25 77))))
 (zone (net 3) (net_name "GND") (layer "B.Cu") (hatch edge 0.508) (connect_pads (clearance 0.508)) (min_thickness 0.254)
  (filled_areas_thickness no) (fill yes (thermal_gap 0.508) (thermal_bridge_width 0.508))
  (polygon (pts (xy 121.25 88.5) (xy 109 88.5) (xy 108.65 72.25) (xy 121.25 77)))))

